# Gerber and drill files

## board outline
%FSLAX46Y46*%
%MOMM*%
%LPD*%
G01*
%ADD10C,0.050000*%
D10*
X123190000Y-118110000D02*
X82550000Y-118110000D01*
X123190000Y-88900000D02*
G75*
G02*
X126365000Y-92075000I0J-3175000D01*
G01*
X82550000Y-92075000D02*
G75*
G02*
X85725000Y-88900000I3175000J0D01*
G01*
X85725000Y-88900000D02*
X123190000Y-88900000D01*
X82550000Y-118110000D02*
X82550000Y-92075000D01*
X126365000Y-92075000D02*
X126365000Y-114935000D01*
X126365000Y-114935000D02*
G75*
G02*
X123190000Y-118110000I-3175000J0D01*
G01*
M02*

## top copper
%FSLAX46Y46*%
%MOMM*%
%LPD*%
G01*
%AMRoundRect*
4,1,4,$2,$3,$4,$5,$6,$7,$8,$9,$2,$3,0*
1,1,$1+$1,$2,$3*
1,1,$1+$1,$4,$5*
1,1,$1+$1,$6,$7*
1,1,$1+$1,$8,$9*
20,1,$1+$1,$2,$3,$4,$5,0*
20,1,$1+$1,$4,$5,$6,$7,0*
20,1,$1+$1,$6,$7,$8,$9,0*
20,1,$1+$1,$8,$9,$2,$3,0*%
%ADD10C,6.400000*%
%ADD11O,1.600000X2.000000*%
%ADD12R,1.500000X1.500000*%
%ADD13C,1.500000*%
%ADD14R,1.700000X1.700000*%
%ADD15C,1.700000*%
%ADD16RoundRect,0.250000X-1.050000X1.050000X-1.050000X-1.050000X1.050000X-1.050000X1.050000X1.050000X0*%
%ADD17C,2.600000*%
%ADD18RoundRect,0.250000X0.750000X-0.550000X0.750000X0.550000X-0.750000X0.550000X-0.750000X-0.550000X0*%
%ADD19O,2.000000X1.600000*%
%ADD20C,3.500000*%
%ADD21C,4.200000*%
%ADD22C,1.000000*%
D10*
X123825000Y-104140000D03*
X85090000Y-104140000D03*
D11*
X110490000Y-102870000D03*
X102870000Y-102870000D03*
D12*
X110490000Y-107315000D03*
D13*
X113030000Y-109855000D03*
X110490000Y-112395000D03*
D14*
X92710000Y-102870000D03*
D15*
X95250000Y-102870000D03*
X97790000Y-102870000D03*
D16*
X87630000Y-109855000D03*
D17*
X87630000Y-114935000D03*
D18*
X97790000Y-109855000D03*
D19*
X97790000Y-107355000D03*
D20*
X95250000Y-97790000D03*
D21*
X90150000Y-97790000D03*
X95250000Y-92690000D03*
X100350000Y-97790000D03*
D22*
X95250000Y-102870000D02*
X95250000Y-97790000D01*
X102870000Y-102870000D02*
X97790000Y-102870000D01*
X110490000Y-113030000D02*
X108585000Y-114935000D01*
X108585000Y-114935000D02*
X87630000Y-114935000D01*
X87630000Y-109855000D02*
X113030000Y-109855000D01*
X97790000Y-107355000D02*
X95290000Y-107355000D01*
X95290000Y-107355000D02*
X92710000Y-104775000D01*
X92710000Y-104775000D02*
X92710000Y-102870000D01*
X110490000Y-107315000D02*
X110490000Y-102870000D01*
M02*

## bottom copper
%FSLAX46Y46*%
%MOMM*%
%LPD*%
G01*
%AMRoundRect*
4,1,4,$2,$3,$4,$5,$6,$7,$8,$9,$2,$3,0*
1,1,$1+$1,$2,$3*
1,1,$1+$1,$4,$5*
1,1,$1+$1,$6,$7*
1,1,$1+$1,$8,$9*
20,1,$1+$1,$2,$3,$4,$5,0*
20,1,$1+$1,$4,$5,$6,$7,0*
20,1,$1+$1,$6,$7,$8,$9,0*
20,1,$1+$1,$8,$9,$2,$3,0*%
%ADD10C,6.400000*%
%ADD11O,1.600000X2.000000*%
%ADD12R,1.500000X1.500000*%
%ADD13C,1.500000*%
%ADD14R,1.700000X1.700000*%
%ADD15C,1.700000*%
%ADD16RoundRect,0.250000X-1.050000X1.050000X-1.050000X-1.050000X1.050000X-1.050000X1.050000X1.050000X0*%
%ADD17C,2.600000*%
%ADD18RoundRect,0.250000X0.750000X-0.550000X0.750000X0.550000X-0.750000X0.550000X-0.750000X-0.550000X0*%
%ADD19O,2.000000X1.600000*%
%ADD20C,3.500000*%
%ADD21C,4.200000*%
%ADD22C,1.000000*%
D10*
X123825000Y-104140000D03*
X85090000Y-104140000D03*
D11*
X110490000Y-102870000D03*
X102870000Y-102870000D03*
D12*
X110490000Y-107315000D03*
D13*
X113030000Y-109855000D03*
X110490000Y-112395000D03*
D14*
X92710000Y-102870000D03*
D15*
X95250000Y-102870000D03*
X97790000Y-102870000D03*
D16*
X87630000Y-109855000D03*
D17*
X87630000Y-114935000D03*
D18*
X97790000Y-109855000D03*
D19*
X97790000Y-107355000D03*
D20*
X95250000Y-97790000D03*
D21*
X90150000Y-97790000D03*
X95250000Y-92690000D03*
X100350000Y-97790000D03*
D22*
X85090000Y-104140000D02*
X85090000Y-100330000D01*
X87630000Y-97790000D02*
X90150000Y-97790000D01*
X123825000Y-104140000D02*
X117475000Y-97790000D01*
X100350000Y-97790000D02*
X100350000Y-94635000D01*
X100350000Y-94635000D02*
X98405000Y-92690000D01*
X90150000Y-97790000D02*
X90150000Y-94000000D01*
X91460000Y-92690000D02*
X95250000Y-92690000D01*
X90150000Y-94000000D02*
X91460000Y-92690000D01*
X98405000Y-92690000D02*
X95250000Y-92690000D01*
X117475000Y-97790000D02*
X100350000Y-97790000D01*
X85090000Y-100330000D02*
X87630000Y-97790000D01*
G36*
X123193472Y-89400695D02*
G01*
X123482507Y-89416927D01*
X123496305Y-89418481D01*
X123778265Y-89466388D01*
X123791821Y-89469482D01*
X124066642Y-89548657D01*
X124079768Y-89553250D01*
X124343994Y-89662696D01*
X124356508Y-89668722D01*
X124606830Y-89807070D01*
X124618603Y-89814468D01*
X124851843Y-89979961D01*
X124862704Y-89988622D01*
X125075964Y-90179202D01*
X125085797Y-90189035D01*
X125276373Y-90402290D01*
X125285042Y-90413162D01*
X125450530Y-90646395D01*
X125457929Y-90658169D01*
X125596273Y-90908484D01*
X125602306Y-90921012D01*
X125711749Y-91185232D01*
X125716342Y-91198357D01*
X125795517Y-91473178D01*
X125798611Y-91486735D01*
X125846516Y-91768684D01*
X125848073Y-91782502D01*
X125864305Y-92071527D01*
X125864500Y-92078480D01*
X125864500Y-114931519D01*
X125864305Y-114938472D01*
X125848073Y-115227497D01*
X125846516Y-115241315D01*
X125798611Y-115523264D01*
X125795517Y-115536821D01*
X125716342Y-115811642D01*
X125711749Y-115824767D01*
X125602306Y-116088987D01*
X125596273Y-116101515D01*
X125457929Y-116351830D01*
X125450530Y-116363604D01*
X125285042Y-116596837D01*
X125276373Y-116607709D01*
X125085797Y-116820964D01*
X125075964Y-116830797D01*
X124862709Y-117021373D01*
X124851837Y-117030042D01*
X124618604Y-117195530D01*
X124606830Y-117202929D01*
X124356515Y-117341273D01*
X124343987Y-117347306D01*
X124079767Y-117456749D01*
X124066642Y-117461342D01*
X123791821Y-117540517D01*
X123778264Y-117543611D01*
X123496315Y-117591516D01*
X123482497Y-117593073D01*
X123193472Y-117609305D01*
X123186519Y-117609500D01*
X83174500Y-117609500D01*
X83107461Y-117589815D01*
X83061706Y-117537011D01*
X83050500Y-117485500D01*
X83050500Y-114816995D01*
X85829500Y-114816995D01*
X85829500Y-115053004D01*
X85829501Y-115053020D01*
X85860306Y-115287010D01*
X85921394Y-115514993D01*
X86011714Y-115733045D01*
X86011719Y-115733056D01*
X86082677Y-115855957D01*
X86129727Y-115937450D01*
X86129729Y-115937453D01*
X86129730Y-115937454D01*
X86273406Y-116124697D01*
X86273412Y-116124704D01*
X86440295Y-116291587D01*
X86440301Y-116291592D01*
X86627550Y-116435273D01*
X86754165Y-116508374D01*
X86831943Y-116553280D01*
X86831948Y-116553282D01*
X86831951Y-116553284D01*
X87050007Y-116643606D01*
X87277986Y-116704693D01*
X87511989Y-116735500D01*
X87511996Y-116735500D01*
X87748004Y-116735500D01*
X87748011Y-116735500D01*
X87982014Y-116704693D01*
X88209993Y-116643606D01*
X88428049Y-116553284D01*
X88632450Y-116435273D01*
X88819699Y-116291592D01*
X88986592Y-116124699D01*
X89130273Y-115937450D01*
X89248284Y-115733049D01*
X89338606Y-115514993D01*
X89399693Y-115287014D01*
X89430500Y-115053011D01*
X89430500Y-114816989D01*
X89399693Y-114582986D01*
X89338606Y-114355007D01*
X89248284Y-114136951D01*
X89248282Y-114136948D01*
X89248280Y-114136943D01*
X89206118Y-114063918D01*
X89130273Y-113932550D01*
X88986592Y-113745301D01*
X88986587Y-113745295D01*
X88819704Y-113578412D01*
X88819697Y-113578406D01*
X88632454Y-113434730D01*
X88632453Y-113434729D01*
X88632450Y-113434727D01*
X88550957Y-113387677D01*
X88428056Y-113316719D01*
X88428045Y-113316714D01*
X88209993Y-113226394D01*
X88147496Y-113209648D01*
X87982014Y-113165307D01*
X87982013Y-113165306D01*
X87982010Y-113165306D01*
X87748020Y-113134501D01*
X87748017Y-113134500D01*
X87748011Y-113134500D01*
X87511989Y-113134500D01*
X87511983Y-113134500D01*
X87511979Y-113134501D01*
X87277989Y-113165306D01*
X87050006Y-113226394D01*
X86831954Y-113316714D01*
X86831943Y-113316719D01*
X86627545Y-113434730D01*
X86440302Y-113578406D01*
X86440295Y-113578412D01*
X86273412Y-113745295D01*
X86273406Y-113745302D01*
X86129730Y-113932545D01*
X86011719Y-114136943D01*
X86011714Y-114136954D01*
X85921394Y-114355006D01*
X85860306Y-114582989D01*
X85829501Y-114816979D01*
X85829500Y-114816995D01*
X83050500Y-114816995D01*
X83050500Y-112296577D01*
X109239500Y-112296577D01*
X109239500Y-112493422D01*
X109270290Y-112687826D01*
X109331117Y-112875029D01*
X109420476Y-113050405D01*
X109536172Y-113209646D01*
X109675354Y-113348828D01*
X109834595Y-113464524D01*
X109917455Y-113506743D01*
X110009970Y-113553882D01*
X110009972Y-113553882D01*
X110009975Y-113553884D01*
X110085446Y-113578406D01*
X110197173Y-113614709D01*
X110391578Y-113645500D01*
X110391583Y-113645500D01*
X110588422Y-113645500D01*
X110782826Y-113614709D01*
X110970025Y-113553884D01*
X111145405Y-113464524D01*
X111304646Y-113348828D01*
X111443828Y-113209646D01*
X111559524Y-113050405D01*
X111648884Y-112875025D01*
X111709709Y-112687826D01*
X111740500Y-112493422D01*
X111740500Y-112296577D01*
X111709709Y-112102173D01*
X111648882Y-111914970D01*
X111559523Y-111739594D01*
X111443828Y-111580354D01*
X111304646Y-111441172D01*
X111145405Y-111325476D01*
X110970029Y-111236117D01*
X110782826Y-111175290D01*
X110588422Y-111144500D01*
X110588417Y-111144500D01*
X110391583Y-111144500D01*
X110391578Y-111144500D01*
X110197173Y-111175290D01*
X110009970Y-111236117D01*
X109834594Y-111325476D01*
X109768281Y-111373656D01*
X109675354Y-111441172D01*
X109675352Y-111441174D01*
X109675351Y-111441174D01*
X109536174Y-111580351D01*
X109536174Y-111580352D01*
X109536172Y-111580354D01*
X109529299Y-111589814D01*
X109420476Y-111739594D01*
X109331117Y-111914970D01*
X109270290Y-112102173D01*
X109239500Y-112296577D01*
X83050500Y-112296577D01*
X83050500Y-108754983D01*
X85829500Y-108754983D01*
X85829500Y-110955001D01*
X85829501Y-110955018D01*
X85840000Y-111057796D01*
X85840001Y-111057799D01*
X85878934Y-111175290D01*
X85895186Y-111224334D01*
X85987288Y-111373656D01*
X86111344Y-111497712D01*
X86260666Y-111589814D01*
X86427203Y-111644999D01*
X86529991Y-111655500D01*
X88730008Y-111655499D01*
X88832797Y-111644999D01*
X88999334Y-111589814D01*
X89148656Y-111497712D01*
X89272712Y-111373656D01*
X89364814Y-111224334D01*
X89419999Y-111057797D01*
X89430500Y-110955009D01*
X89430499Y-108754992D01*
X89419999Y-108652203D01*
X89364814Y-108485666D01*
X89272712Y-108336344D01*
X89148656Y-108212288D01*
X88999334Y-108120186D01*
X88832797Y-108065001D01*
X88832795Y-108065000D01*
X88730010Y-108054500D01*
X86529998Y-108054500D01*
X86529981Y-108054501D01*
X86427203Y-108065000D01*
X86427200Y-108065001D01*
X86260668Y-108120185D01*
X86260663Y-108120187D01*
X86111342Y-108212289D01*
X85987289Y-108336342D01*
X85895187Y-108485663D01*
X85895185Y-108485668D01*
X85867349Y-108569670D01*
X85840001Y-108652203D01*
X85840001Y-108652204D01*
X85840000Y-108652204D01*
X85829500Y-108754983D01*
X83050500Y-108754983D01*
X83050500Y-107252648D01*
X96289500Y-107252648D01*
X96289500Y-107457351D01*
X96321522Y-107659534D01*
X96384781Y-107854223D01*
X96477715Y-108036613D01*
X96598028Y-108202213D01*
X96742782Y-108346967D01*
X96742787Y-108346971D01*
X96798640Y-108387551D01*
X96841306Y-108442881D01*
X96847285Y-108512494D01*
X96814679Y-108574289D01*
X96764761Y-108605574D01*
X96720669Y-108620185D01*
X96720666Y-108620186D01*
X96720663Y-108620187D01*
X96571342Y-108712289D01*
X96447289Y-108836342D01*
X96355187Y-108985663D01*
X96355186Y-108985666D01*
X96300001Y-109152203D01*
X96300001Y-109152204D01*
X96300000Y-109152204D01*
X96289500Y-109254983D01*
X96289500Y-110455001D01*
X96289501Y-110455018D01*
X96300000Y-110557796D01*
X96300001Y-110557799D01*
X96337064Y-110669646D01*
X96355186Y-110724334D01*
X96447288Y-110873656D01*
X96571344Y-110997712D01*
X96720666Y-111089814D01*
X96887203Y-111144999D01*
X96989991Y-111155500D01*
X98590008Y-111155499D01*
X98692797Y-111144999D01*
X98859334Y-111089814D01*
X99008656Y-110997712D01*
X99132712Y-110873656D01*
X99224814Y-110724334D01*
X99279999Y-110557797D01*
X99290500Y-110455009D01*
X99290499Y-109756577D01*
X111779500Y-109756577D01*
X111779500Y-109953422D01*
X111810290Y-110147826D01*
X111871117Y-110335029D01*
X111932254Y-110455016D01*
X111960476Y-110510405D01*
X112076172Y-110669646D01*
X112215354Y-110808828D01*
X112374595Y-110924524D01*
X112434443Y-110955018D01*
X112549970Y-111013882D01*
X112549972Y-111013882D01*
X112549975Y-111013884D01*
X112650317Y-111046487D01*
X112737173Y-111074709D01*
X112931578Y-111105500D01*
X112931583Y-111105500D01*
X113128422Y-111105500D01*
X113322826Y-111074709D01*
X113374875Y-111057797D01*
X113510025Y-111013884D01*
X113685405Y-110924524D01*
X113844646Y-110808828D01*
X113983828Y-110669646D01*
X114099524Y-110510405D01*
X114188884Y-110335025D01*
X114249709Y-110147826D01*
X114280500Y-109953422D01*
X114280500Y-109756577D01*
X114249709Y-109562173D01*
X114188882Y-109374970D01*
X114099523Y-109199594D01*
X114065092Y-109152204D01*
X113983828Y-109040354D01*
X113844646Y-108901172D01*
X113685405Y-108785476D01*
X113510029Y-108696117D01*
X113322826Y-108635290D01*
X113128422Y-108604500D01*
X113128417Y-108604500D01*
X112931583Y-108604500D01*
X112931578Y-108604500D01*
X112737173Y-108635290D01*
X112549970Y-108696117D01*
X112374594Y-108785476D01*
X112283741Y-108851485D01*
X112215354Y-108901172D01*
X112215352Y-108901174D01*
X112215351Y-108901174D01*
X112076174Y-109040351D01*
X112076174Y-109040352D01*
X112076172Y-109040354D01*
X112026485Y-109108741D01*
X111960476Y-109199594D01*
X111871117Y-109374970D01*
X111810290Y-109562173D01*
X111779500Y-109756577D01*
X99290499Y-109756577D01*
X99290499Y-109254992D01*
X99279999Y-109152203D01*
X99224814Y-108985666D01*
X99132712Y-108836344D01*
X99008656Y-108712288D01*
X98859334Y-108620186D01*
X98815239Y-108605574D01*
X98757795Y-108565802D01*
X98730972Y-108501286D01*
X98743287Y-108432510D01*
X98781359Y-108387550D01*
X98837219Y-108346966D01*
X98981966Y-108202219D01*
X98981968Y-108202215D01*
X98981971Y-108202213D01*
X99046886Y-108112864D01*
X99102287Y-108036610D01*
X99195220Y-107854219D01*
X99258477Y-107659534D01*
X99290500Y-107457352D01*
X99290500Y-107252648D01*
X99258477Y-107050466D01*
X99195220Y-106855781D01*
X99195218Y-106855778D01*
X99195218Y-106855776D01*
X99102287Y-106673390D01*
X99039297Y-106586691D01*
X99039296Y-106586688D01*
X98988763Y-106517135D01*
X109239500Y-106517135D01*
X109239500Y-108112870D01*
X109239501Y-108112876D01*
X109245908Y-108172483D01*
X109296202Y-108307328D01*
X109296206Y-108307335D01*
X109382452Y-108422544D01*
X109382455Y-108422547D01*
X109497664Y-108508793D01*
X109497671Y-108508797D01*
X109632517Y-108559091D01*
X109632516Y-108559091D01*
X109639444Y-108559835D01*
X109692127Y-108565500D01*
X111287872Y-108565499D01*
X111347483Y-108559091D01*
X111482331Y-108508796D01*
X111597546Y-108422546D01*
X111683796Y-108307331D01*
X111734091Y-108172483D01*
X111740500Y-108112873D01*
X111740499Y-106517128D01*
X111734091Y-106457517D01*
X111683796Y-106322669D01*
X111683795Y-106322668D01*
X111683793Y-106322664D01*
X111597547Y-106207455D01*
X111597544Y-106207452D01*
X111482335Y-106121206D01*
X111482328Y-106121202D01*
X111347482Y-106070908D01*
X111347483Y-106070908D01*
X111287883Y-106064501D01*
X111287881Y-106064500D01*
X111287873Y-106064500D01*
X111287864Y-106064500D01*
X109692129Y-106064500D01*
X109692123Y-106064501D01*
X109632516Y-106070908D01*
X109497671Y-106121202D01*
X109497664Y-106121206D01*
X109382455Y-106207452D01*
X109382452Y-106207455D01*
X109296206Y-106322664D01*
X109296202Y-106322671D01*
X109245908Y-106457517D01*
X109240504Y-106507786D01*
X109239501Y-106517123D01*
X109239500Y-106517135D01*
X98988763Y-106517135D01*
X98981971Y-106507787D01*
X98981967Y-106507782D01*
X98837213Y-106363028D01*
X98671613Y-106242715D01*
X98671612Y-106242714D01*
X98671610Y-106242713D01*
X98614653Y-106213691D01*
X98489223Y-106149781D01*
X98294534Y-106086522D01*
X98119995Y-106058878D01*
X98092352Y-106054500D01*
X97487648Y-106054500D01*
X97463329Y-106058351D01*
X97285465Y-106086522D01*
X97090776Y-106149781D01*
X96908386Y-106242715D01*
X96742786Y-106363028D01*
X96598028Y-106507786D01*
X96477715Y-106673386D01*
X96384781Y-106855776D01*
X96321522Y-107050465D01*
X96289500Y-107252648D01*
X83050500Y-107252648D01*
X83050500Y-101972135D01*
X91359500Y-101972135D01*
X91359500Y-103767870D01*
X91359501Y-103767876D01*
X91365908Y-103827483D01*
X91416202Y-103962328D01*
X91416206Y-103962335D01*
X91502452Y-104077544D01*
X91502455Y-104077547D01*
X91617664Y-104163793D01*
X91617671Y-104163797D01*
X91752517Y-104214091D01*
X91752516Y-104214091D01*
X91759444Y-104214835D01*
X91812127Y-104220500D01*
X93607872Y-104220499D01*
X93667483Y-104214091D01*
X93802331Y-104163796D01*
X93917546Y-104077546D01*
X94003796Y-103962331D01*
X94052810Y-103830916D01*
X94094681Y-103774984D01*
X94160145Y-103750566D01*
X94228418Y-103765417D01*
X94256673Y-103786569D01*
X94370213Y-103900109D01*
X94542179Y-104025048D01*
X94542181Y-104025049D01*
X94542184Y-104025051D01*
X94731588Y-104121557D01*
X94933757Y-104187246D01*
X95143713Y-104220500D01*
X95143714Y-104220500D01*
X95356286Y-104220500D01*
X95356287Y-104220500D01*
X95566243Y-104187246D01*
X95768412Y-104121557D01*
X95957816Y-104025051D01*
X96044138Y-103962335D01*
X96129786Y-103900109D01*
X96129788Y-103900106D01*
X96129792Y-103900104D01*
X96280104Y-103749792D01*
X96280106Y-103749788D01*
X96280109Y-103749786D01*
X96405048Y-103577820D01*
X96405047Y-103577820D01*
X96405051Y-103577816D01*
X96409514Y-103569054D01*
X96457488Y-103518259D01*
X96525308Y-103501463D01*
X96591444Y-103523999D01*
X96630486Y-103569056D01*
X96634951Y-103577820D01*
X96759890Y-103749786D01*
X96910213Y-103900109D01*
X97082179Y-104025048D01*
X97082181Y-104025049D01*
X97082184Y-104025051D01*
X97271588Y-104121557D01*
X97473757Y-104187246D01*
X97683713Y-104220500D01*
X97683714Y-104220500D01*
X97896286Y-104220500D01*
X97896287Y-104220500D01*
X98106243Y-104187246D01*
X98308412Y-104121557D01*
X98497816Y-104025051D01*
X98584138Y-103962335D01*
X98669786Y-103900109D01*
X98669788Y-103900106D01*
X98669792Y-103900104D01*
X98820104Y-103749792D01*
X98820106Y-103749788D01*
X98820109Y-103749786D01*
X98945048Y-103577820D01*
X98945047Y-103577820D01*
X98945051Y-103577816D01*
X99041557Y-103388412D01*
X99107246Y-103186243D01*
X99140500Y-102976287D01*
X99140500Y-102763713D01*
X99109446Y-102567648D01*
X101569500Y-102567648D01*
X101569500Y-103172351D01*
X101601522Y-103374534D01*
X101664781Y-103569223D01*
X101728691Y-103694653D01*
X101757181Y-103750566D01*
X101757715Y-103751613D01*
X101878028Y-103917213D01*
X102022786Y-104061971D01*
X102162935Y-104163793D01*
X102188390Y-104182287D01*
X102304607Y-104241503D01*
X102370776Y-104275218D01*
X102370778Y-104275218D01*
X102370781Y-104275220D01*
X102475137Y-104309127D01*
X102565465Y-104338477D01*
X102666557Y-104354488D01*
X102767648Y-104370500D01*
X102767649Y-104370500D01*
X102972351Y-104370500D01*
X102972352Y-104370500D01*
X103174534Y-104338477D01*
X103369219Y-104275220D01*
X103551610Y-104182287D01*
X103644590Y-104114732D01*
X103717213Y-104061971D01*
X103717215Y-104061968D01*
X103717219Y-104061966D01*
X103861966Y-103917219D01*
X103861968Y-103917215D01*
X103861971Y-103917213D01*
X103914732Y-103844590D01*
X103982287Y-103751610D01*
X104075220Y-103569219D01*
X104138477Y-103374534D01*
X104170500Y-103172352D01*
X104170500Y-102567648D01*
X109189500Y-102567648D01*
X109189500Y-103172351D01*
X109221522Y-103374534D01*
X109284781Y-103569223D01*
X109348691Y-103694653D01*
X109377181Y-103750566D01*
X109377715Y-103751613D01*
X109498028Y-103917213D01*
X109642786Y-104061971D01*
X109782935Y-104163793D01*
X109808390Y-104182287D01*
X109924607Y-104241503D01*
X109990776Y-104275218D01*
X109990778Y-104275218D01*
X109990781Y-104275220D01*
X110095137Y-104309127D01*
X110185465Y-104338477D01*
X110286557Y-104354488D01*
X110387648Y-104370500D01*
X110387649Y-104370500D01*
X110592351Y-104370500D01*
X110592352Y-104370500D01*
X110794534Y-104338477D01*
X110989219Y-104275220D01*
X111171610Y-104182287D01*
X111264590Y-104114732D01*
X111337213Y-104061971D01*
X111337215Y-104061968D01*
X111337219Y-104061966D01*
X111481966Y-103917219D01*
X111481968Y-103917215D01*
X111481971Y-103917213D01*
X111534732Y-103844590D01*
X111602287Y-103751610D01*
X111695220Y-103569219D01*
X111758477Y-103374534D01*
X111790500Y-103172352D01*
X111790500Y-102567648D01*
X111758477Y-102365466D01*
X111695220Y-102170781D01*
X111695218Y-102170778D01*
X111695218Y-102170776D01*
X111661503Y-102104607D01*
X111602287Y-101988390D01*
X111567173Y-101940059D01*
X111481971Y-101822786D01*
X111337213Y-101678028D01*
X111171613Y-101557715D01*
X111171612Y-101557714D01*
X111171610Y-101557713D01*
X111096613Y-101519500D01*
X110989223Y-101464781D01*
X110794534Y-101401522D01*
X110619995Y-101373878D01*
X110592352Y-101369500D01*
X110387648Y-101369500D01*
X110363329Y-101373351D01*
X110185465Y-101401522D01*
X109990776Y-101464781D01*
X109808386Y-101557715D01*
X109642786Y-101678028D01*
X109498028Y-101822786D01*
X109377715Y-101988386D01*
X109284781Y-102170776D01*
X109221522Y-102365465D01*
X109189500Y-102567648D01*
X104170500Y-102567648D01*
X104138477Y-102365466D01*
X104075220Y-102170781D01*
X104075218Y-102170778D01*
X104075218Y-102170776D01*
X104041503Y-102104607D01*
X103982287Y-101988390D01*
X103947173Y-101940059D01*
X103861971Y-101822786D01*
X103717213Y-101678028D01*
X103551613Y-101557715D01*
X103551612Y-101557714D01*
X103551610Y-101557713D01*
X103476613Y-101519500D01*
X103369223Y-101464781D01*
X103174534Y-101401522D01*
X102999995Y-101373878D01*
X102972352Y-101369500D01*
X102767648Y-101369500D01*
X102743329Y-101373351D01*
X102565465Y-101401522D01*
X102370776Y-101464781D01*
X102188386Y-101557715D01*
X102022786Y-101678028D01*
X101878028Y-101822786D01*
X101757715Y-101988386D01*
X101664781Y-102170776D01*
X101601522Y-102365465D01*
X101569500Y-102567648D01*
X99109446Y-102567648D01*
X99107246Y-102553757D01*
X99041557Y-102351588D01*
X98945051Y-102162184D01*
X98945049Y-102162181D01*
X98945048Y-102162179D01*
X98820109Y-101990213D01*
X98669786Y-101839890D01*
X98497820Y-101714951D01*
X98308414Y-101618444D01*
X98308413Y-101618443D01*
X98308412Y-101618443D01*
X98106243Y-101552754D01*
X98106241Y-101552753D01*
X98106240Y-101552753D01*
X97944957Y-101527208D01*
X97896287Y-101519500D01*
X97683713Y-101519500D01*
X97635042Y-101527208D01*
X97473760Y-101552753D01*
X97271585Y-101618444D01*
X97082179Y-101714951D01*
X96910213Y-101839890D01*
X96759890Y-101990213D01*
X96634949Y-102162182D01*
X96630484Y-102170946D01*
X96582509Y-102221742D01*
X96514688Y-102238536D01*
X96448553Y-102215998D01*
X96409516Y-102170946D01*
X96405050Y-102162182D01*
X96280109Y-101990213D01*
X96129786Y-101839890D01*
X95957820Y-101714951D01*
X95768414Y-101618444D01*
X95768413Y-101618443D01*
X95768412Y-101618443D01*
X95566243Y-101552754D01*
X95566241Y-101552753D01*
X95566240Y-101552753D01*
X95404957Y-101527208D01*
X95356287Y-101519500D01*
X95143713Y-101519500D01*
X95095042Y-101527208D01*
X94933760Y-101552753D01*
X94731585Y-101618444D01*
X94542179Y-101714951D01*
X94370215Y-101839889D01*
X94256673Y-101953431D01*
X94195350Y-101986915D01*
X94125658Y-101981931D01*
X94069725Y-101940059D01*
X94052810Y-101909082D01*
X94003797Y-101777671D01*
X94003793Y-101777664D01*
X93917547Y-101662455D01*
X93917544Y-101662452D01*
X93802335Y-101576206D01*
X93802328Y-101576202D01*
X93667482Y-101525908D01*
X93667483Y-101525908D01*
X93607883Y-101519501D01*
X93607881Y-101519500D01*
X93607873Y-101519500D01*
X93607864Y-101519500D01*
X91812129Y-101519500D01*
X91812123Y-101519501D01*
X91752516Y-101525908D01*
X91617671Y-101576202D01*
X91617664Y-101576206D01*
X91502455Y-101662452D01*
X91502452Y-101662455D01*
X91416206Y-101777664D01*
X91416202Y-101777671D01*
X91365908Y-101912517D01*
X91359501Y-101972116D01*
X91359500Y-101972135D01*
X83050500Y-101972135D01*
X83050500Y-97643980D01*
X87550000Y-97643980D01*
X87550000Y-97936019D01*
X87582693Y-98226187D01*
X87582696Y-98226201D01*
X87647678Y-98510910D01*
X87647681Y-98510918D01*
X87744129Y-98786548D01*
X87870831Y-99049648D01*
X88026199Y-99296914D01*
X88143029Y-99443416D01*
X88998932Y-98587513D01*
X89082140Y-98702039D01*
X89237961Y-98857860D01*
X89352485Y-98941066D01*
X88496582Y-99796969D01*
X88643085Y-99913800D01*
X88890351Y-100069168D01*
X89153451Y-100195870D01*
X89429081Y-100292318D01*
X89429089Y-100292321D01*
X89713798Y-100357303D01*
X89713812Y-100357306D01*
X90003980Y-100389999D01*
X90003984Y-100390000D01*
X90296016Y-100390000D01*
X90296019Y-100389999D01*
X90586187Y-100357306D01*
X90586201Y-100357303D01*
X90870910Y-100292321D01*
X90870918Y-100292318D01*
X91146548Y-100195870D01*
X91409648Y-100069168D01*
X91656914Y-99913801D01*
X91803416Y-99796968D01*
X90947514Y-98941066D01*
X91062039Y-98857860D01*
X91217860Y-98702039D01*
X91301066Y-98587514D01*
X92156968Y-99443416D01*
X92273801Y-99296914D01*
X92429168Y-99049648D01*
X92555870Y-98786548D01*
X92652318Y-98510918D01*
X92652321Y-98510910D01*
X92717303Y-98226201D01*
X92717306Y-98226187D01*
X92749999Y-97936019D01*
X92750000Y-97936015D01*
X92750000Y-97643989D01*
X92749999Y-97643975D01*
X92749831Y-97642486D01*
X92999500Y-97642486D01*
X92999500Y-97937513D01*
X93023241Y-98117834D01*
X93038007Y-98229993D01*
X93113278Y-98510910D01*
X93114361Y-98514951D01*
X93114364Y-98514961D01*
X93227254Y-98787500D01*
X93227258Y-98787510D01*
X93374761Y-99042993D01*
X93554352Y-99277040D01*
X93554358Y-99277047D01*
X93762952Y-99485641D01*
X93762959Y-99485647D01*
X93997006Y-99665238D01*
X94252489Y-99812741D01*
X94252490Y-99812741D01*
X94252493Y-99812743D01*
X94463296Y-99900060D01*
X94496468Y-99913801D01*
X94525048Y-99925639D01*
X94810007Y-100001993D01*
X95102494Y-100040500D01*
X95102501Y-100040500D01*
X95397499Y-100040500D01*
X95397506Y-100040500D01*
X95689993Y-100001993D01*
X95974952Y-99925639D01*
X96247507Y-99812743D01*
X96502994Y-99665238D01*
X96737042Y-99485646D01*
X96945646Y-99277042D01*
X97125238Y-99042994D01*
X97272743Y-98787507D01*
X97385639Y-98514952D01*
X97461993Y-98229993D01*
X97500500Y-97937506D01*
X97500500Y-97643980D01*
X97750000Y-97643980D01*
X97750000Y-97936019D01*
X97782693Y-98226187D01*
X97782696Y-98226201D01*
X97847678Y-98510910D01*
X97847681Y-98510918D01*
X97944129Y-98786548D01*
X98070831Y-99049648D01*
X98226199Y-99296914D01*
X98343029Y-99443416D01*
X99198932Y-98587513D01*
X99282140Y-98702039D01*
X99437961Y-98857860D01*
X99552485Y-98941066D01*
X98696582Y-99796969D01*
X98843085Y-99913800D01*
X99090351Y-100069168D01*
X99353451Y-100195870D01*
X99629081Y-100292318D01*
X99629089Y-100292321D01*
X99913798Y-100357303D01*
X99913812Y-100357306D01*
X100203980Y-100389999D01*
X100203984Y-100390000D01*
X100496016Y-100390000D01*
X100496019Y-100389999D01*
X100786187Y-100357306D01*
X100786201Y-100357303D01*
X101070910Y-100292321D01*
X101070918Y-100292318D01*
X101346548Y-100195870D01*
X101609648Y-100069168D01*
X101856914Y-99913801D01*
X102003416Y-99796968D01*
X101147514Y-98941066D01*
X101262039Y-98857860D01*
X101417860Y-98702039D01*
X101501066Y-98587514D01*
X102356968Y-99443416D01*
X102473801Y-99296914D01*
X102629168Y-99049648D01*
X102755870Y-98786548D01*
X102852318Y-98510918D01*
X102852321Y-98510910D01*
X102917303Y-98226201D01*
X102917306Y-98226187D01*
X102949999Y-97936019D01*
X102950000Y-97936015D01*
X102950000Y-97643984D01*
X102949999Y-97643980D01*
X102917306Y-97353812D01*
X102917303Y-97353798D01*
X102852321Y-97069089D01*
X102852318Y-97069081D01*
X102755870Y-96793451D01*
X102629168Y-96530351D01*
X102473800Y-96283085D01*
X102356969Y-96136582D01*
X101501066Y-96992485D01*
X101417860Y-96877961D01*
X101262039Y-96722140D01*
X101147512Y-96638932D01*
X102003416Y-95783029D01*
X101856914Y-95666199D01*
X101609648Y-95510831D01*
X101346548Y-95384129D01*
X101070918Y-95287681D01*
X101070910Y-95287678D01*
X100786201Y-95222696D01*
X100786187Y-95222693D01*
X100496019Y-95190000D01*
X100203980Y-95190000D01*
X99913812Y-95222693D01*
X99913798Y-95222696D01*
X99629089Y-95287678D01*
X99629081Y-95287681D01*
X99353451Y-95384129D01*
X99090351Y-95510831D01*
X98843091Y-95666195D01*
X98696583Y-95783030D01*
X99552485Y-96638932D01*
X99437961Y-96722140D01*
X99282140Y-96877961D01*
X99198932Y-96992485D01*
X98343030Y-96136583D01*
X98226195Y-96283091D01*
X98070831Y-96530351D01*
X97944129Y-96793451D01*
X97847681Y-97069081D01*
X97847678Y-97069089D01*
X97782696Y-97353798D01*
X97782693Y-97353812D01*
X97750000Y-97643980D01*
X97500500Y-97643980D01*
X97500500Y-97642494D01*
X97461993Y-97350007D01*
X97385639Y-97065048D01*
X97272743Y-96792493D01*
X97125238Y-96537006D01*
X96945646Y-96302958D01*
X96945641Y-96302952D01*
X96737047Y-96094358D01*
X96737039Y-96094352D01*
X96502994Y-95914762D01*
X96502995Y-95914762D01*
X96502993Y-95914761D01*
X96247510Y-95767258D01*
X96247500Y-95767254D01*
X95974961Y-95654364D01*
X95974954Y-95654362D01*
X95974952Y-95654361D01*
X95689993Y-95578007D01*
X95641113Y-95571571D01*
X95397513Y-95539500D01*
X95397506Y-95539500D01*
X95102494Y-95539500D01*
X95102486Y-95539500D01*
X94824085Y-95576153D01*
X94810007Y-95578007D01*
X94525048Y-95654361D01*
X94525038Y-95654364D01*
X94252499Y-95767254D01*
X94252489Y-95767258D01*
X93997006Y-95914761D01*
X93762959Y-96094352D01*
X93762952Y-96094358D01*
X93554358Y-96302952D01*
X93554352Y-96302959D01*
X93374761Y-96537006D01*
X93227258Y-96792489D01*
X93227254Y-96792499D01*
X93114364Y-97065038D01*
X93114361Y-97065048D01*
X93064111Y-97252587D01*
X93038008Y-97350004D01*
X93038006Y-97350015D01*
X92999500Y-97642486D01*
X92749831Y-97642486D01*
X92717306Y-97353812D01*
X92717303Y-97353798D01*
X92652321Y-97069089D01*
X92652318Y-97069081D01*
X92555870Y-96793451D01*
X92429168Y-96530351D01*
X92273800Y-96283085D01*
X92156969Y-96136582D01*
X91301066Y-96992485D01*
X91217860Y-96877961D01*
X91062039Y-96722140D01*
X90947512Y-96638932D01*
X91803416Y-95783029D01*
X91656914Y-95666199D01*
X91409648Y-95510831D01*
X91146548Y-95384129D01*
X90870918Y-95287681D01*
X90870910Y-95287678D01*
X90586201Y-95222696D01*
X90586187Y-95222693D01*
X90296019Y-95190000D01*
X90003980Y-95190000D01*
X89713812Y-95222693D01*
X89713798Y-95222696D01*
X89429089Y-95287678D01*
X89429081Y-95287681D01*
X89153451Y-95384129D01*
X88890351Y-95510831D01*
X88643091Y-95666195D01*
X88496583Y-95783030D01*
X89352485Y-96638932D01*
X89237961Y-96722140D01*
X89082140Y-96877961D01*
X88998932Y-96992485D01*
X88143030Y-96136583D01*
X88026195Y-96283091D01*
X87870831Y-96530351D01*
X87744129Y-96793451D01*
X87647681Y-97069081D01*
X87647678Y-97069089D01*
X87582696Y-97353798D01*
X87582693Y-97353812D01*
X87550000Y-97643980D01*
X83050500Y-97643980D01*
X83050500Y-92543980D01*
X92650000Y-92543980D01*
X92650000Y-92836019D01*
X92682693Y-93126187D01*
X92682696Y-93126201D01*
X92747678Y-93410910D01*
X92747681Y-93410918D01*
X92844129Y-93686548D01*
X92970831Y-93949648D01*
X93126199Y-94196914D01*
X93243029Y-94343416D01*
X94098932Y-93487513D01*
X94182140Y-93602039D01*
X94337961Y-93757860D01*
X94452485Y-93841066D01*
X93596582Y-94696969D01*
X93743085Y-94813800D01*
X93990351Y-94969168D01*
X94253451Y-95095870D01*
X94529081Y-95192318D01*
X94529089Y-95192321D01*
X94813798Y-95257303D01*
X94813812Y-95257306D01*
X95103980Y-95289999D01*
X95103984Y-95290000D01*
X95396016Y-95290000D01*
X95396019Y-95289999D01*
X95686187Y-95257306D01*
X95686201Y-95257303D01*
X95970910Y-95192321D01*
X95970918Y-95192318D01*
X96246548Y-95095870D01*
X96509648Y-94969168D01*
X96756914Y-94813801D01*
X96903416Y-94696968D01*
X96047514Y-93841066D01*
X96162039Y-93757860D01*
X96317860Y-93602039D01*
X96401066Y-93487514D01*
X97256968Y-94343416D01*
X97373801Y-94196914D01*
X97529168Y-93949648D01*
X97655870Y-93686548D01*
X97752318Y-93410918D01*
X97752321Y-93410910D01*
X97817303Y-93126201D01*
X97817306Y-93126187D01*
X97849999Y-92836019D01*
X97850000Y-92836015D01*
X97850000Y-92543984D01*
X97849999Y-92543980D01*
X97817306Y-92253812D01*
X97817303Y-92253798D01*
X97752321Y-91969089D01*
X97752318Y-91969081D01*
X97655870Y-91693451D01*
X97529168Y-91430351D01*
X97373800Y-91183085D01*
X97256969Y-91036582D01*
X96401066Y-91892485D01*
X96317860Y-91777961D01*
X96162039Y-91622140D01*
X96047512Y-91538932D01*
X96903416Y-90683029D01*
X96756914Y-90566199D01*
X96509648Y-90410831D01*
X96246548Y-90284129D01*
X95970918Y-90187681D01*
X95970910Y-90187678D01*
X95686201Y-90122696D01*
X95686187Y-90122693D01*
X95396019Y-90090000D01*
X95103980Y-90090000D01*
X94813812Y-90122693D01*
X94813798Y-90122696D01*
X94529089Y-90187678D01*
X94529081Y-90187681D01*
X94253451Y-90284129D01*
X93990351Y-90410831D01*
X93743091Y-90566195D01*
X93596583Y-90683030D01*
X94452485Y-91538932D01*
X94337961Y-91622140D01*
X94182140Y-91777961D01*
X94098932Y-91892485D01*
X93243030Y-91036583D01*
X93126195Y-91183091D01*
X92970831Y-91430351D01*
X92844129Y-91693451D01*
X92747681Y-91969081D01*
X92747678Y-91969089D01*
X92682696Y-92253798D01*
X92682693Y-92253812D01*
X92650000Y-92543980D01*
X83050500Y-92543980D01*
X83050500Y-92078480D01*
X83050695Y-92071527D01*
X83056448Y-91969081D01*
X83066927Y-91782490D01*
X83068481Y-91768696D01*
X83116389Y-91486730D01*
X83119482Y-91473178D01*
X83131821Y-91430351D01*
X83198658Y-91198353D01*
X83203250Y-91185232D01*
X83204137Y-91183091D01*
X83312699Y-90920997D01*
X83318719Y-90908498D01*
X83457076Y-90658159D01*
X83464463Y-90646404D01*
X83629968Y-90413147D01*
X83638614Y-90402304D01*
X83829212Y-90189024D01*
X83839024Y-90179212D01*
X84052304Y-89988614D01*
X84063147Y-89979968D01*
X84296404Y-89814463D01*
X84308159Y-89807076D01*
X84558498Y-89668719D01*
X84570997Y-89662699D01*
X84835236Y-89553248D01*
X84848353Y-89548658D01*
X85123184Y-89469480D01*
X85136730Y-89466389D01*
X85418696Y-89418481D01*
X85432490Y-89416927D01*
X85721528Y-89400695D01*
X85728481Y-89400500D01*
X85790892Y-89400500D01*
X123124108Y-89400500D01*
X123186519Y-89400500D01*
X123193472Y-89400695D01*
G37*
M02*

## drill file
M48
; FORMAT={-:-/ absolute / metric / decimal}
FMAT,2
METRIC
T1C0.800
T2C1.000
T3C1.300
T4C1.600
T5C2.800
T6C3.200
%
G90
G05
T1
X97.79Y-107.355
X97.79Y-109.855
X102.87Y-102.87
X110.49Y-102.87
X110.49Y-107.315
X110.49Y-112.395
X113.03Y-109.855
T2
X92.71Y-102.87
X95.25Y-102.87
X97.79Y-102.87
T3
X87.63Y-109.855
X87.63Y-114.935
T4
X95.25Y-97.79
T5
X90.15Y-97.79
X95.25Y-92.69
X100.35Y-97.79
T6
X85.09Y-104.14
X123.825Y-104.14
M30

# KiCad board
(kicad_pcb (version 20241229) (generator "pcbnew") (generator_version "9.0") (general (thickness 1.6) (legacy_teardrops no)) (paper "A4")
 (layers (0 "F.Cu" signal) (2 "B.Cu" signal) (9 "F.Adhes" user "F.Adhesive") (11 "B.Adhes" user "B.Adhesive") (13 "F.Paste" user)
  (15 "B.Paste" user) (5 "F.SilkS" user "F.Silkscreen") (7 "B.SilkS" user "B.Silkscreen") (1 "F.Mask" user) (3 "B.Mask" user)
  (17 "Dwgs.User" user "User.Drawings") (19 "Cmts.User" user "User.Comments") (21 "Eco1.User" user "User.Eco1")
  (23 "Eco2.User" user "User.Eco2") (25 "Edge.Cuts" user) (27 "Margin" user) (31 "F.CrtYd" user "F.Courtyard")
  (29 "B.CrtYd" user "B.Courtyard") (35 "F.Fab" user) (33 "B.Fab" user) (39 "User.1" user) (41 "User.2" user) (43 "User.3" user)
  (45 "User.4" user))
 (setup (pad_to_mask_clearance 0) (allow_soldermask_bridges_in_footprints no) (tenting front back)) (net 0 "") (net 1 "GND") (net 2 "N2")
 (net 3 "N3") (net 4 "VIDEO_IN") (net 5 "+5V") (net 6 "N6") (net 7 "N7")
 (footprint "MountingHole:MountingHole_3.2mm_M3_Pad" (layer "F.Cu") (at 123.825 104.14)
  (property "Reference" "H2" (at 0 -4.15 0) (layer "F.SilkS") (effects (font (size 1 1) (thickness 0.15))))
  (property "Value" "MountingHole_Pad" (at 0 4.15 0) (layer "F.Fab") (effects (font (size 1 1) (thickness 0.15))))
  (pad "1" thru_hole circle (at 0 0) (size 6.4 6.4) (drill 3.2) (layers "*.Cu" "*.Mask") (remove_unused_layers no) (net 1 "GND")
   (zone_connect 2)))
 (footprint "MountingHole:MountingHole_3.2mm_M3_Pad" (layer "F.Cu") (at 85.09 104.14)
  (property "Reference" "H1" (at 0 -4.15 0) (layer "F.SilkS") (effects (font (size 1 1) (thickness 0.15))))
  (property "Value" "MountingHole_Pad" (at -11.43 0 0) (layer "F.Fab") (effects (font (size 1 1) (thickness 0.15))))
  (pad "1" thru_hole circle (at 0 0) (size 6.4 6.4) (drill 3.2) (layers "*.Cu" "*.Mask") (remove_unused_layers no) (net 1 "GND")
   (zone_connect 2)))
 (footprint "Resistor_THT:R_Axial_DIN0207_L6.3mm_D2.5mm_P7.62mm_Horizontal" (layer "F.Cu") (at 110.49 102.87 180)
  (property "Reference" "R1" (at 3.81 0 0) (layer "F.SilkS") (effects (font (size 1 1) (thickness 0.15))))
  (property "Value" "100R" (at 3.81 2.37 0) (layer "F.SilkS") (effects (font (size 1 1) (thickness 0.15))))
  (pad "1" thru_hole oval (at 0 0 180) (size 1.6 2) (drill 0.8) (layers "*.Cu" "*.Mask") (remove_unused_layers no) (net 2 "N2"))
  (pad "2" thru_hole oval (at 7.62 0 180) (size 1.6 2) (drill 0.8) (layers "*.Cu" "*.Mask") (remove_unused_layers no) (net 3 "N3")))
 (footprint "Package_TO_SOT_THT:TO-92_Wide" (layer "F.Cu") (at 110.49 107.315 -90)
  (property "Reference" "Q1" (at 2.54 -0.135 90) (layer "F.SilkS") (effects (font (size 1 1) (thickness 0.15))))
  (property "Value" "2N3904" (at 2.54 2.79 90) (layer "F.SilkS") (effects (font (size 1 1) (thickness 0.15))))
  (pad "1" thru_hole rect (at 0 0 270) (size 1.5 1.5) (drill 0.8) (layers "*.Cu" "*.Mask") (remove_unused_layers no) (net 2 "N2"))
  (pad "2" thru_hole circle (at 2.54 -2.54 270) (size 1.5 1.5) (drill 0.8) (layers "*.Cu" "*.Mask") (remove_unused_layers no)
   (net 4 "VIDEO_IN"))
  (pad "3" thru_hole circle (at 5.08 0 270) (size 1.5 1.5) (drill 0.8) (layers "*.Cu" "*.Mask") (remove_unused_layers no) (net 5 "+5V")))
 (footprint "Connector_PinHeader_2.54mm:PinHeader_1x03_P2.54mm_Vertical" (layer "F.Cu") (at 92.71 102.87 90)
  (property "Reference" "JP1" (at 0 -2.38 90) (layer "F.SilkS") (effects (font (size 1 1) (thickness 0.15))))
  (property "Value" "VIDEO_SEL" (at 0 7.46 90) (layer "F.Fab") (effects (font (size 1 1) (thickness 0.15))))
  (pad "1" thru_hole rect (at 0 0 90) (size 1.7 1.7) (drill 1) (layers "*.Cu" "*.Mask") (remove_unused_layers no) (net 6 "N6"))
  (pad "2" thru_hole circle (at 0 2.54 90) (size 1.7 1.7) (drill 1) (layers "*.Cu" "*.Mask") (remove_unused_layers no) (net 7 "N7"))
  (pad "3" thru_hole circle (at 0 5.08 90) (size 1.7 1.7) (drill 1) (layers "*.Cu" "*.Mask") (remove_unused_layers no) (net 3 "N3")))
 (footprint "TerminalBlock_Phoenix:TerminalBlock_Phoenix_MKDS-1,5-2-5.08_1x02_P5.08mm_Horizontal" (layer "F.Cu") (at 87.63 109.855 -90)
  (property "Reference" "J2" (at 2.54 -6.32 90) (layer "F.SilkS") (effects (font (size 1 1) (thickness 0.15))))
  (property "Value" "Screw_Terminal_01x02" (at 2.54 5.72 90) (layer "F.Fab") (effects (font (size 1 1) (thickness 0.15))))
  (pad "1" thru_hole roundrect (at 0 0 270) (size 2.6 2.6) (drill 1.3) (layers "*.Cu" "*.Mask") (remove_unused_layers no)
   (roundrect_rratio 0.096154) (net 4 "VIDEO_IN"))
  (pad "2" thru_hole circle (at 5.08 0 270) (size 2.6 2.6) (drill 1.3) (layers "*.Cu" "*.Mask") (remove_unused_layers no) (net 5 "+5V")))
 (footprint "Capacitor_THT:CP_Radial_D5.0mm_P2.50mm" (layer "F.Cu") (at 97.79 109.855 90)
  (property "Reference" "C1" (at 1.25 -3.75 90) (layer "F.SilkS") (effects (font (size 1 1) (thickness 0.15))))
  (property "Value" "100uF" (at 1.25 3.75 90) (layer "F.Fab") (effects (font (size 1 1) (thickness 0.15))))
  (pad "1" thru_hole roundrect (at 0 0 90) (size 1.6 2) (drill 0.8) (layers "*.Cu" "*.Mask") (remove_unused_layers no)
   (roundrect_rratio 0.15625) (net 4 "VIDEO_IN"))
  (pad "2" thru_hole oval (at 2.5 0 90) (size 1.6 2) (drill 0.8) (layers "*.Cu" "*.Mask") (remove_unused_layers no) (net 6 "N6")))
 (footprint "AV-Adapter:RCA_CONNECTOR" (layer "F.Cu") (at 95.25 97.79)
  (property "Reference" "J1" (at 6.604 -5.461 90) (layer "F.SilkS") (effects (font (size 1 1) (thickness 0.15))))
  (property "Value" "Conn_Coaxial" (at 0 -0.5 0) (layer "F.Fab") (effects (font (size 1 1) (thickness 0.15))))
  (pad "1" thru_hole circle (at 0 0) (size 3.5 3.5) (drill 1.6) (layers "*.Cu" "*.Mask") (remove_unused_layers no) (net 7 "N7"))
  (pad "2" thru_hole circle (at -5.1 0) (size 4.2 4.2) (drill 2.8) (layers "*.Cu" "*.Mask") (remove_unused_layers no) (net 1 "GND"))
  (pad "2" thru_hole circle (at 0 -5.1) (size 4.2 4.2) (drill 2.8) (layers "*.Cu" "*.Mask") (remove_unused_layers no) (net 1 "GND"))
  (pad "2" thru_hole circle (at 5.1 0) (size 4.2 4.2) (drill 2.8) (layers "*.Cu" "*.Mask") (remove_unused_layers no) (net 1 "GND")))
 (gr_line (start 123.19 118.11) (end 82.55 118.11) (stroke (width 0.05) (type default)) (layer "Edge.Cuts"))
 (gr_arc (start 123.19 88.9) (mid 125.435064 89.829936) (end 126.365 92.075) (stroke (width 0.05) (type default)) (layer "Edge.Cuts"))
 (gr_arc (start 82.55 92.075) (mid 83.479936 89.829936) (end 85.725 88.9) (stroke (width 0.05) (type default)) (layer "Edge.Cuts"))
 (gr_line (start 85.725 88.9) (end 123.19 88.9) (stroke (width 0.05) (type default)) (layer "Edge.Cuts"))
 (gr_line (start 82.55 118.11) (end 82.55 92.075) (stroke (width 0.05) (type default)) (layer "Edge.Cuts"))
 (gr_line (start 126.365 92.075) (end 126.365 114.935) (stroke (width 0.05) (type default)) (layer "Edge.Cuts"))
 (gr_arc (start 126.365 114.935) (mid 125.435064 117.180064) (end 123.19 118.11) (stroke (width 0.05) (type default)) (layer "Edge.Cuts"))
 (segment (start 85.09 104.14) (end 85.09 100.33) (width 1) (layer "B.Cu") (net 1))
 (segment (start 87.63 97.79) (end 90.15 97.79) (width 1) (layer "B.Cu") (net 1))
 (segment (start 123.825 104.14) (end 117.475 97.79) (width 1) (layer "B.Cu") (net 1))
 (segment (start 100.35 97.79) (end 100.35 94.635) (width 1) (layer "B.Cu") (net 1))
 (segment (start 100.35 94.635) (end 98.405 92.69) (width 1) (layer "B.Cu") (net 1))
 (segment (start 90.15 97.79) (end 90.15 94) (width 1) (layer "B.Cu") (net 1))
 (segment (start 91.46 92.69) (end 95.25 92.69) (width 1) (layer "B.Cu") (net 1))
 (segment (start 90.15 94) (end 91.46 92.69) (width 1) (layer "B.Cu") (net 1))
 (segment (start 98.405 92.69) (end 95.25 92.69) (width 1) (layer "B.Cu") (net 1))
 (segment (start 117.475 97.79) (end 100.35 97.79) (width 1) (layer "B.Cu") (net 1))
 (segment (start 85.09 100.33) (end 87.63 97.79) (width 1) (layer "B.Cu") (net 1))
 (segment (start 95.25 102.87) (end 95.25 97.79) (width 1) (layer "F.Cu") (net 7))
 (segment (start 102.87 102.87) (end 97.79 102.87) (width 1) (layer "F.Cu") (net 3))
 (segment (start 110.49 113.03) (end 108.585 114.935) (width 1) (layer "F.Cu") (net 5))
 (segment (start 108.585 114.935) (end 87.63 114.935) (width 1) (layer "F.Cu") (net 5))
 (segment (start 87.63 109.855) (end 113.03 109.855) (width 1) (layer "F.Cu") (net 4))
 (segment (start 97.79 107.355) (end 95.29 107.355) (width 1) (layer "F.Cu") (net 6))
 (segment (start 95.29 107.355) (end 92.71 104.775) (width 1) (layer "F.Cu") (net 6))
 (segment (start 92.71 104.775) (end 92.71 102.87) (width 1) (layer "F.Cu") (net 6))
 (segment (start 110.49 107.315) (end 110.49 102.87) (width 1) (layer "F.Cu") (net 2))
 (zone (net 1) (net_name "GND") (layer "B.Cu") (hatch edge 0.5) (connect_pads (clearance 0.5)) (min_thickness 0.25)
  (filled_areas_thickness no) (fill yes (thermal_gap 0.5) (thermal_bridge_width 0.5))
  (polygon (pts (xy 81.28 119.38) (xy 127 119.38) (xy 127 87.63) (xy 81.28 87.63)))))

